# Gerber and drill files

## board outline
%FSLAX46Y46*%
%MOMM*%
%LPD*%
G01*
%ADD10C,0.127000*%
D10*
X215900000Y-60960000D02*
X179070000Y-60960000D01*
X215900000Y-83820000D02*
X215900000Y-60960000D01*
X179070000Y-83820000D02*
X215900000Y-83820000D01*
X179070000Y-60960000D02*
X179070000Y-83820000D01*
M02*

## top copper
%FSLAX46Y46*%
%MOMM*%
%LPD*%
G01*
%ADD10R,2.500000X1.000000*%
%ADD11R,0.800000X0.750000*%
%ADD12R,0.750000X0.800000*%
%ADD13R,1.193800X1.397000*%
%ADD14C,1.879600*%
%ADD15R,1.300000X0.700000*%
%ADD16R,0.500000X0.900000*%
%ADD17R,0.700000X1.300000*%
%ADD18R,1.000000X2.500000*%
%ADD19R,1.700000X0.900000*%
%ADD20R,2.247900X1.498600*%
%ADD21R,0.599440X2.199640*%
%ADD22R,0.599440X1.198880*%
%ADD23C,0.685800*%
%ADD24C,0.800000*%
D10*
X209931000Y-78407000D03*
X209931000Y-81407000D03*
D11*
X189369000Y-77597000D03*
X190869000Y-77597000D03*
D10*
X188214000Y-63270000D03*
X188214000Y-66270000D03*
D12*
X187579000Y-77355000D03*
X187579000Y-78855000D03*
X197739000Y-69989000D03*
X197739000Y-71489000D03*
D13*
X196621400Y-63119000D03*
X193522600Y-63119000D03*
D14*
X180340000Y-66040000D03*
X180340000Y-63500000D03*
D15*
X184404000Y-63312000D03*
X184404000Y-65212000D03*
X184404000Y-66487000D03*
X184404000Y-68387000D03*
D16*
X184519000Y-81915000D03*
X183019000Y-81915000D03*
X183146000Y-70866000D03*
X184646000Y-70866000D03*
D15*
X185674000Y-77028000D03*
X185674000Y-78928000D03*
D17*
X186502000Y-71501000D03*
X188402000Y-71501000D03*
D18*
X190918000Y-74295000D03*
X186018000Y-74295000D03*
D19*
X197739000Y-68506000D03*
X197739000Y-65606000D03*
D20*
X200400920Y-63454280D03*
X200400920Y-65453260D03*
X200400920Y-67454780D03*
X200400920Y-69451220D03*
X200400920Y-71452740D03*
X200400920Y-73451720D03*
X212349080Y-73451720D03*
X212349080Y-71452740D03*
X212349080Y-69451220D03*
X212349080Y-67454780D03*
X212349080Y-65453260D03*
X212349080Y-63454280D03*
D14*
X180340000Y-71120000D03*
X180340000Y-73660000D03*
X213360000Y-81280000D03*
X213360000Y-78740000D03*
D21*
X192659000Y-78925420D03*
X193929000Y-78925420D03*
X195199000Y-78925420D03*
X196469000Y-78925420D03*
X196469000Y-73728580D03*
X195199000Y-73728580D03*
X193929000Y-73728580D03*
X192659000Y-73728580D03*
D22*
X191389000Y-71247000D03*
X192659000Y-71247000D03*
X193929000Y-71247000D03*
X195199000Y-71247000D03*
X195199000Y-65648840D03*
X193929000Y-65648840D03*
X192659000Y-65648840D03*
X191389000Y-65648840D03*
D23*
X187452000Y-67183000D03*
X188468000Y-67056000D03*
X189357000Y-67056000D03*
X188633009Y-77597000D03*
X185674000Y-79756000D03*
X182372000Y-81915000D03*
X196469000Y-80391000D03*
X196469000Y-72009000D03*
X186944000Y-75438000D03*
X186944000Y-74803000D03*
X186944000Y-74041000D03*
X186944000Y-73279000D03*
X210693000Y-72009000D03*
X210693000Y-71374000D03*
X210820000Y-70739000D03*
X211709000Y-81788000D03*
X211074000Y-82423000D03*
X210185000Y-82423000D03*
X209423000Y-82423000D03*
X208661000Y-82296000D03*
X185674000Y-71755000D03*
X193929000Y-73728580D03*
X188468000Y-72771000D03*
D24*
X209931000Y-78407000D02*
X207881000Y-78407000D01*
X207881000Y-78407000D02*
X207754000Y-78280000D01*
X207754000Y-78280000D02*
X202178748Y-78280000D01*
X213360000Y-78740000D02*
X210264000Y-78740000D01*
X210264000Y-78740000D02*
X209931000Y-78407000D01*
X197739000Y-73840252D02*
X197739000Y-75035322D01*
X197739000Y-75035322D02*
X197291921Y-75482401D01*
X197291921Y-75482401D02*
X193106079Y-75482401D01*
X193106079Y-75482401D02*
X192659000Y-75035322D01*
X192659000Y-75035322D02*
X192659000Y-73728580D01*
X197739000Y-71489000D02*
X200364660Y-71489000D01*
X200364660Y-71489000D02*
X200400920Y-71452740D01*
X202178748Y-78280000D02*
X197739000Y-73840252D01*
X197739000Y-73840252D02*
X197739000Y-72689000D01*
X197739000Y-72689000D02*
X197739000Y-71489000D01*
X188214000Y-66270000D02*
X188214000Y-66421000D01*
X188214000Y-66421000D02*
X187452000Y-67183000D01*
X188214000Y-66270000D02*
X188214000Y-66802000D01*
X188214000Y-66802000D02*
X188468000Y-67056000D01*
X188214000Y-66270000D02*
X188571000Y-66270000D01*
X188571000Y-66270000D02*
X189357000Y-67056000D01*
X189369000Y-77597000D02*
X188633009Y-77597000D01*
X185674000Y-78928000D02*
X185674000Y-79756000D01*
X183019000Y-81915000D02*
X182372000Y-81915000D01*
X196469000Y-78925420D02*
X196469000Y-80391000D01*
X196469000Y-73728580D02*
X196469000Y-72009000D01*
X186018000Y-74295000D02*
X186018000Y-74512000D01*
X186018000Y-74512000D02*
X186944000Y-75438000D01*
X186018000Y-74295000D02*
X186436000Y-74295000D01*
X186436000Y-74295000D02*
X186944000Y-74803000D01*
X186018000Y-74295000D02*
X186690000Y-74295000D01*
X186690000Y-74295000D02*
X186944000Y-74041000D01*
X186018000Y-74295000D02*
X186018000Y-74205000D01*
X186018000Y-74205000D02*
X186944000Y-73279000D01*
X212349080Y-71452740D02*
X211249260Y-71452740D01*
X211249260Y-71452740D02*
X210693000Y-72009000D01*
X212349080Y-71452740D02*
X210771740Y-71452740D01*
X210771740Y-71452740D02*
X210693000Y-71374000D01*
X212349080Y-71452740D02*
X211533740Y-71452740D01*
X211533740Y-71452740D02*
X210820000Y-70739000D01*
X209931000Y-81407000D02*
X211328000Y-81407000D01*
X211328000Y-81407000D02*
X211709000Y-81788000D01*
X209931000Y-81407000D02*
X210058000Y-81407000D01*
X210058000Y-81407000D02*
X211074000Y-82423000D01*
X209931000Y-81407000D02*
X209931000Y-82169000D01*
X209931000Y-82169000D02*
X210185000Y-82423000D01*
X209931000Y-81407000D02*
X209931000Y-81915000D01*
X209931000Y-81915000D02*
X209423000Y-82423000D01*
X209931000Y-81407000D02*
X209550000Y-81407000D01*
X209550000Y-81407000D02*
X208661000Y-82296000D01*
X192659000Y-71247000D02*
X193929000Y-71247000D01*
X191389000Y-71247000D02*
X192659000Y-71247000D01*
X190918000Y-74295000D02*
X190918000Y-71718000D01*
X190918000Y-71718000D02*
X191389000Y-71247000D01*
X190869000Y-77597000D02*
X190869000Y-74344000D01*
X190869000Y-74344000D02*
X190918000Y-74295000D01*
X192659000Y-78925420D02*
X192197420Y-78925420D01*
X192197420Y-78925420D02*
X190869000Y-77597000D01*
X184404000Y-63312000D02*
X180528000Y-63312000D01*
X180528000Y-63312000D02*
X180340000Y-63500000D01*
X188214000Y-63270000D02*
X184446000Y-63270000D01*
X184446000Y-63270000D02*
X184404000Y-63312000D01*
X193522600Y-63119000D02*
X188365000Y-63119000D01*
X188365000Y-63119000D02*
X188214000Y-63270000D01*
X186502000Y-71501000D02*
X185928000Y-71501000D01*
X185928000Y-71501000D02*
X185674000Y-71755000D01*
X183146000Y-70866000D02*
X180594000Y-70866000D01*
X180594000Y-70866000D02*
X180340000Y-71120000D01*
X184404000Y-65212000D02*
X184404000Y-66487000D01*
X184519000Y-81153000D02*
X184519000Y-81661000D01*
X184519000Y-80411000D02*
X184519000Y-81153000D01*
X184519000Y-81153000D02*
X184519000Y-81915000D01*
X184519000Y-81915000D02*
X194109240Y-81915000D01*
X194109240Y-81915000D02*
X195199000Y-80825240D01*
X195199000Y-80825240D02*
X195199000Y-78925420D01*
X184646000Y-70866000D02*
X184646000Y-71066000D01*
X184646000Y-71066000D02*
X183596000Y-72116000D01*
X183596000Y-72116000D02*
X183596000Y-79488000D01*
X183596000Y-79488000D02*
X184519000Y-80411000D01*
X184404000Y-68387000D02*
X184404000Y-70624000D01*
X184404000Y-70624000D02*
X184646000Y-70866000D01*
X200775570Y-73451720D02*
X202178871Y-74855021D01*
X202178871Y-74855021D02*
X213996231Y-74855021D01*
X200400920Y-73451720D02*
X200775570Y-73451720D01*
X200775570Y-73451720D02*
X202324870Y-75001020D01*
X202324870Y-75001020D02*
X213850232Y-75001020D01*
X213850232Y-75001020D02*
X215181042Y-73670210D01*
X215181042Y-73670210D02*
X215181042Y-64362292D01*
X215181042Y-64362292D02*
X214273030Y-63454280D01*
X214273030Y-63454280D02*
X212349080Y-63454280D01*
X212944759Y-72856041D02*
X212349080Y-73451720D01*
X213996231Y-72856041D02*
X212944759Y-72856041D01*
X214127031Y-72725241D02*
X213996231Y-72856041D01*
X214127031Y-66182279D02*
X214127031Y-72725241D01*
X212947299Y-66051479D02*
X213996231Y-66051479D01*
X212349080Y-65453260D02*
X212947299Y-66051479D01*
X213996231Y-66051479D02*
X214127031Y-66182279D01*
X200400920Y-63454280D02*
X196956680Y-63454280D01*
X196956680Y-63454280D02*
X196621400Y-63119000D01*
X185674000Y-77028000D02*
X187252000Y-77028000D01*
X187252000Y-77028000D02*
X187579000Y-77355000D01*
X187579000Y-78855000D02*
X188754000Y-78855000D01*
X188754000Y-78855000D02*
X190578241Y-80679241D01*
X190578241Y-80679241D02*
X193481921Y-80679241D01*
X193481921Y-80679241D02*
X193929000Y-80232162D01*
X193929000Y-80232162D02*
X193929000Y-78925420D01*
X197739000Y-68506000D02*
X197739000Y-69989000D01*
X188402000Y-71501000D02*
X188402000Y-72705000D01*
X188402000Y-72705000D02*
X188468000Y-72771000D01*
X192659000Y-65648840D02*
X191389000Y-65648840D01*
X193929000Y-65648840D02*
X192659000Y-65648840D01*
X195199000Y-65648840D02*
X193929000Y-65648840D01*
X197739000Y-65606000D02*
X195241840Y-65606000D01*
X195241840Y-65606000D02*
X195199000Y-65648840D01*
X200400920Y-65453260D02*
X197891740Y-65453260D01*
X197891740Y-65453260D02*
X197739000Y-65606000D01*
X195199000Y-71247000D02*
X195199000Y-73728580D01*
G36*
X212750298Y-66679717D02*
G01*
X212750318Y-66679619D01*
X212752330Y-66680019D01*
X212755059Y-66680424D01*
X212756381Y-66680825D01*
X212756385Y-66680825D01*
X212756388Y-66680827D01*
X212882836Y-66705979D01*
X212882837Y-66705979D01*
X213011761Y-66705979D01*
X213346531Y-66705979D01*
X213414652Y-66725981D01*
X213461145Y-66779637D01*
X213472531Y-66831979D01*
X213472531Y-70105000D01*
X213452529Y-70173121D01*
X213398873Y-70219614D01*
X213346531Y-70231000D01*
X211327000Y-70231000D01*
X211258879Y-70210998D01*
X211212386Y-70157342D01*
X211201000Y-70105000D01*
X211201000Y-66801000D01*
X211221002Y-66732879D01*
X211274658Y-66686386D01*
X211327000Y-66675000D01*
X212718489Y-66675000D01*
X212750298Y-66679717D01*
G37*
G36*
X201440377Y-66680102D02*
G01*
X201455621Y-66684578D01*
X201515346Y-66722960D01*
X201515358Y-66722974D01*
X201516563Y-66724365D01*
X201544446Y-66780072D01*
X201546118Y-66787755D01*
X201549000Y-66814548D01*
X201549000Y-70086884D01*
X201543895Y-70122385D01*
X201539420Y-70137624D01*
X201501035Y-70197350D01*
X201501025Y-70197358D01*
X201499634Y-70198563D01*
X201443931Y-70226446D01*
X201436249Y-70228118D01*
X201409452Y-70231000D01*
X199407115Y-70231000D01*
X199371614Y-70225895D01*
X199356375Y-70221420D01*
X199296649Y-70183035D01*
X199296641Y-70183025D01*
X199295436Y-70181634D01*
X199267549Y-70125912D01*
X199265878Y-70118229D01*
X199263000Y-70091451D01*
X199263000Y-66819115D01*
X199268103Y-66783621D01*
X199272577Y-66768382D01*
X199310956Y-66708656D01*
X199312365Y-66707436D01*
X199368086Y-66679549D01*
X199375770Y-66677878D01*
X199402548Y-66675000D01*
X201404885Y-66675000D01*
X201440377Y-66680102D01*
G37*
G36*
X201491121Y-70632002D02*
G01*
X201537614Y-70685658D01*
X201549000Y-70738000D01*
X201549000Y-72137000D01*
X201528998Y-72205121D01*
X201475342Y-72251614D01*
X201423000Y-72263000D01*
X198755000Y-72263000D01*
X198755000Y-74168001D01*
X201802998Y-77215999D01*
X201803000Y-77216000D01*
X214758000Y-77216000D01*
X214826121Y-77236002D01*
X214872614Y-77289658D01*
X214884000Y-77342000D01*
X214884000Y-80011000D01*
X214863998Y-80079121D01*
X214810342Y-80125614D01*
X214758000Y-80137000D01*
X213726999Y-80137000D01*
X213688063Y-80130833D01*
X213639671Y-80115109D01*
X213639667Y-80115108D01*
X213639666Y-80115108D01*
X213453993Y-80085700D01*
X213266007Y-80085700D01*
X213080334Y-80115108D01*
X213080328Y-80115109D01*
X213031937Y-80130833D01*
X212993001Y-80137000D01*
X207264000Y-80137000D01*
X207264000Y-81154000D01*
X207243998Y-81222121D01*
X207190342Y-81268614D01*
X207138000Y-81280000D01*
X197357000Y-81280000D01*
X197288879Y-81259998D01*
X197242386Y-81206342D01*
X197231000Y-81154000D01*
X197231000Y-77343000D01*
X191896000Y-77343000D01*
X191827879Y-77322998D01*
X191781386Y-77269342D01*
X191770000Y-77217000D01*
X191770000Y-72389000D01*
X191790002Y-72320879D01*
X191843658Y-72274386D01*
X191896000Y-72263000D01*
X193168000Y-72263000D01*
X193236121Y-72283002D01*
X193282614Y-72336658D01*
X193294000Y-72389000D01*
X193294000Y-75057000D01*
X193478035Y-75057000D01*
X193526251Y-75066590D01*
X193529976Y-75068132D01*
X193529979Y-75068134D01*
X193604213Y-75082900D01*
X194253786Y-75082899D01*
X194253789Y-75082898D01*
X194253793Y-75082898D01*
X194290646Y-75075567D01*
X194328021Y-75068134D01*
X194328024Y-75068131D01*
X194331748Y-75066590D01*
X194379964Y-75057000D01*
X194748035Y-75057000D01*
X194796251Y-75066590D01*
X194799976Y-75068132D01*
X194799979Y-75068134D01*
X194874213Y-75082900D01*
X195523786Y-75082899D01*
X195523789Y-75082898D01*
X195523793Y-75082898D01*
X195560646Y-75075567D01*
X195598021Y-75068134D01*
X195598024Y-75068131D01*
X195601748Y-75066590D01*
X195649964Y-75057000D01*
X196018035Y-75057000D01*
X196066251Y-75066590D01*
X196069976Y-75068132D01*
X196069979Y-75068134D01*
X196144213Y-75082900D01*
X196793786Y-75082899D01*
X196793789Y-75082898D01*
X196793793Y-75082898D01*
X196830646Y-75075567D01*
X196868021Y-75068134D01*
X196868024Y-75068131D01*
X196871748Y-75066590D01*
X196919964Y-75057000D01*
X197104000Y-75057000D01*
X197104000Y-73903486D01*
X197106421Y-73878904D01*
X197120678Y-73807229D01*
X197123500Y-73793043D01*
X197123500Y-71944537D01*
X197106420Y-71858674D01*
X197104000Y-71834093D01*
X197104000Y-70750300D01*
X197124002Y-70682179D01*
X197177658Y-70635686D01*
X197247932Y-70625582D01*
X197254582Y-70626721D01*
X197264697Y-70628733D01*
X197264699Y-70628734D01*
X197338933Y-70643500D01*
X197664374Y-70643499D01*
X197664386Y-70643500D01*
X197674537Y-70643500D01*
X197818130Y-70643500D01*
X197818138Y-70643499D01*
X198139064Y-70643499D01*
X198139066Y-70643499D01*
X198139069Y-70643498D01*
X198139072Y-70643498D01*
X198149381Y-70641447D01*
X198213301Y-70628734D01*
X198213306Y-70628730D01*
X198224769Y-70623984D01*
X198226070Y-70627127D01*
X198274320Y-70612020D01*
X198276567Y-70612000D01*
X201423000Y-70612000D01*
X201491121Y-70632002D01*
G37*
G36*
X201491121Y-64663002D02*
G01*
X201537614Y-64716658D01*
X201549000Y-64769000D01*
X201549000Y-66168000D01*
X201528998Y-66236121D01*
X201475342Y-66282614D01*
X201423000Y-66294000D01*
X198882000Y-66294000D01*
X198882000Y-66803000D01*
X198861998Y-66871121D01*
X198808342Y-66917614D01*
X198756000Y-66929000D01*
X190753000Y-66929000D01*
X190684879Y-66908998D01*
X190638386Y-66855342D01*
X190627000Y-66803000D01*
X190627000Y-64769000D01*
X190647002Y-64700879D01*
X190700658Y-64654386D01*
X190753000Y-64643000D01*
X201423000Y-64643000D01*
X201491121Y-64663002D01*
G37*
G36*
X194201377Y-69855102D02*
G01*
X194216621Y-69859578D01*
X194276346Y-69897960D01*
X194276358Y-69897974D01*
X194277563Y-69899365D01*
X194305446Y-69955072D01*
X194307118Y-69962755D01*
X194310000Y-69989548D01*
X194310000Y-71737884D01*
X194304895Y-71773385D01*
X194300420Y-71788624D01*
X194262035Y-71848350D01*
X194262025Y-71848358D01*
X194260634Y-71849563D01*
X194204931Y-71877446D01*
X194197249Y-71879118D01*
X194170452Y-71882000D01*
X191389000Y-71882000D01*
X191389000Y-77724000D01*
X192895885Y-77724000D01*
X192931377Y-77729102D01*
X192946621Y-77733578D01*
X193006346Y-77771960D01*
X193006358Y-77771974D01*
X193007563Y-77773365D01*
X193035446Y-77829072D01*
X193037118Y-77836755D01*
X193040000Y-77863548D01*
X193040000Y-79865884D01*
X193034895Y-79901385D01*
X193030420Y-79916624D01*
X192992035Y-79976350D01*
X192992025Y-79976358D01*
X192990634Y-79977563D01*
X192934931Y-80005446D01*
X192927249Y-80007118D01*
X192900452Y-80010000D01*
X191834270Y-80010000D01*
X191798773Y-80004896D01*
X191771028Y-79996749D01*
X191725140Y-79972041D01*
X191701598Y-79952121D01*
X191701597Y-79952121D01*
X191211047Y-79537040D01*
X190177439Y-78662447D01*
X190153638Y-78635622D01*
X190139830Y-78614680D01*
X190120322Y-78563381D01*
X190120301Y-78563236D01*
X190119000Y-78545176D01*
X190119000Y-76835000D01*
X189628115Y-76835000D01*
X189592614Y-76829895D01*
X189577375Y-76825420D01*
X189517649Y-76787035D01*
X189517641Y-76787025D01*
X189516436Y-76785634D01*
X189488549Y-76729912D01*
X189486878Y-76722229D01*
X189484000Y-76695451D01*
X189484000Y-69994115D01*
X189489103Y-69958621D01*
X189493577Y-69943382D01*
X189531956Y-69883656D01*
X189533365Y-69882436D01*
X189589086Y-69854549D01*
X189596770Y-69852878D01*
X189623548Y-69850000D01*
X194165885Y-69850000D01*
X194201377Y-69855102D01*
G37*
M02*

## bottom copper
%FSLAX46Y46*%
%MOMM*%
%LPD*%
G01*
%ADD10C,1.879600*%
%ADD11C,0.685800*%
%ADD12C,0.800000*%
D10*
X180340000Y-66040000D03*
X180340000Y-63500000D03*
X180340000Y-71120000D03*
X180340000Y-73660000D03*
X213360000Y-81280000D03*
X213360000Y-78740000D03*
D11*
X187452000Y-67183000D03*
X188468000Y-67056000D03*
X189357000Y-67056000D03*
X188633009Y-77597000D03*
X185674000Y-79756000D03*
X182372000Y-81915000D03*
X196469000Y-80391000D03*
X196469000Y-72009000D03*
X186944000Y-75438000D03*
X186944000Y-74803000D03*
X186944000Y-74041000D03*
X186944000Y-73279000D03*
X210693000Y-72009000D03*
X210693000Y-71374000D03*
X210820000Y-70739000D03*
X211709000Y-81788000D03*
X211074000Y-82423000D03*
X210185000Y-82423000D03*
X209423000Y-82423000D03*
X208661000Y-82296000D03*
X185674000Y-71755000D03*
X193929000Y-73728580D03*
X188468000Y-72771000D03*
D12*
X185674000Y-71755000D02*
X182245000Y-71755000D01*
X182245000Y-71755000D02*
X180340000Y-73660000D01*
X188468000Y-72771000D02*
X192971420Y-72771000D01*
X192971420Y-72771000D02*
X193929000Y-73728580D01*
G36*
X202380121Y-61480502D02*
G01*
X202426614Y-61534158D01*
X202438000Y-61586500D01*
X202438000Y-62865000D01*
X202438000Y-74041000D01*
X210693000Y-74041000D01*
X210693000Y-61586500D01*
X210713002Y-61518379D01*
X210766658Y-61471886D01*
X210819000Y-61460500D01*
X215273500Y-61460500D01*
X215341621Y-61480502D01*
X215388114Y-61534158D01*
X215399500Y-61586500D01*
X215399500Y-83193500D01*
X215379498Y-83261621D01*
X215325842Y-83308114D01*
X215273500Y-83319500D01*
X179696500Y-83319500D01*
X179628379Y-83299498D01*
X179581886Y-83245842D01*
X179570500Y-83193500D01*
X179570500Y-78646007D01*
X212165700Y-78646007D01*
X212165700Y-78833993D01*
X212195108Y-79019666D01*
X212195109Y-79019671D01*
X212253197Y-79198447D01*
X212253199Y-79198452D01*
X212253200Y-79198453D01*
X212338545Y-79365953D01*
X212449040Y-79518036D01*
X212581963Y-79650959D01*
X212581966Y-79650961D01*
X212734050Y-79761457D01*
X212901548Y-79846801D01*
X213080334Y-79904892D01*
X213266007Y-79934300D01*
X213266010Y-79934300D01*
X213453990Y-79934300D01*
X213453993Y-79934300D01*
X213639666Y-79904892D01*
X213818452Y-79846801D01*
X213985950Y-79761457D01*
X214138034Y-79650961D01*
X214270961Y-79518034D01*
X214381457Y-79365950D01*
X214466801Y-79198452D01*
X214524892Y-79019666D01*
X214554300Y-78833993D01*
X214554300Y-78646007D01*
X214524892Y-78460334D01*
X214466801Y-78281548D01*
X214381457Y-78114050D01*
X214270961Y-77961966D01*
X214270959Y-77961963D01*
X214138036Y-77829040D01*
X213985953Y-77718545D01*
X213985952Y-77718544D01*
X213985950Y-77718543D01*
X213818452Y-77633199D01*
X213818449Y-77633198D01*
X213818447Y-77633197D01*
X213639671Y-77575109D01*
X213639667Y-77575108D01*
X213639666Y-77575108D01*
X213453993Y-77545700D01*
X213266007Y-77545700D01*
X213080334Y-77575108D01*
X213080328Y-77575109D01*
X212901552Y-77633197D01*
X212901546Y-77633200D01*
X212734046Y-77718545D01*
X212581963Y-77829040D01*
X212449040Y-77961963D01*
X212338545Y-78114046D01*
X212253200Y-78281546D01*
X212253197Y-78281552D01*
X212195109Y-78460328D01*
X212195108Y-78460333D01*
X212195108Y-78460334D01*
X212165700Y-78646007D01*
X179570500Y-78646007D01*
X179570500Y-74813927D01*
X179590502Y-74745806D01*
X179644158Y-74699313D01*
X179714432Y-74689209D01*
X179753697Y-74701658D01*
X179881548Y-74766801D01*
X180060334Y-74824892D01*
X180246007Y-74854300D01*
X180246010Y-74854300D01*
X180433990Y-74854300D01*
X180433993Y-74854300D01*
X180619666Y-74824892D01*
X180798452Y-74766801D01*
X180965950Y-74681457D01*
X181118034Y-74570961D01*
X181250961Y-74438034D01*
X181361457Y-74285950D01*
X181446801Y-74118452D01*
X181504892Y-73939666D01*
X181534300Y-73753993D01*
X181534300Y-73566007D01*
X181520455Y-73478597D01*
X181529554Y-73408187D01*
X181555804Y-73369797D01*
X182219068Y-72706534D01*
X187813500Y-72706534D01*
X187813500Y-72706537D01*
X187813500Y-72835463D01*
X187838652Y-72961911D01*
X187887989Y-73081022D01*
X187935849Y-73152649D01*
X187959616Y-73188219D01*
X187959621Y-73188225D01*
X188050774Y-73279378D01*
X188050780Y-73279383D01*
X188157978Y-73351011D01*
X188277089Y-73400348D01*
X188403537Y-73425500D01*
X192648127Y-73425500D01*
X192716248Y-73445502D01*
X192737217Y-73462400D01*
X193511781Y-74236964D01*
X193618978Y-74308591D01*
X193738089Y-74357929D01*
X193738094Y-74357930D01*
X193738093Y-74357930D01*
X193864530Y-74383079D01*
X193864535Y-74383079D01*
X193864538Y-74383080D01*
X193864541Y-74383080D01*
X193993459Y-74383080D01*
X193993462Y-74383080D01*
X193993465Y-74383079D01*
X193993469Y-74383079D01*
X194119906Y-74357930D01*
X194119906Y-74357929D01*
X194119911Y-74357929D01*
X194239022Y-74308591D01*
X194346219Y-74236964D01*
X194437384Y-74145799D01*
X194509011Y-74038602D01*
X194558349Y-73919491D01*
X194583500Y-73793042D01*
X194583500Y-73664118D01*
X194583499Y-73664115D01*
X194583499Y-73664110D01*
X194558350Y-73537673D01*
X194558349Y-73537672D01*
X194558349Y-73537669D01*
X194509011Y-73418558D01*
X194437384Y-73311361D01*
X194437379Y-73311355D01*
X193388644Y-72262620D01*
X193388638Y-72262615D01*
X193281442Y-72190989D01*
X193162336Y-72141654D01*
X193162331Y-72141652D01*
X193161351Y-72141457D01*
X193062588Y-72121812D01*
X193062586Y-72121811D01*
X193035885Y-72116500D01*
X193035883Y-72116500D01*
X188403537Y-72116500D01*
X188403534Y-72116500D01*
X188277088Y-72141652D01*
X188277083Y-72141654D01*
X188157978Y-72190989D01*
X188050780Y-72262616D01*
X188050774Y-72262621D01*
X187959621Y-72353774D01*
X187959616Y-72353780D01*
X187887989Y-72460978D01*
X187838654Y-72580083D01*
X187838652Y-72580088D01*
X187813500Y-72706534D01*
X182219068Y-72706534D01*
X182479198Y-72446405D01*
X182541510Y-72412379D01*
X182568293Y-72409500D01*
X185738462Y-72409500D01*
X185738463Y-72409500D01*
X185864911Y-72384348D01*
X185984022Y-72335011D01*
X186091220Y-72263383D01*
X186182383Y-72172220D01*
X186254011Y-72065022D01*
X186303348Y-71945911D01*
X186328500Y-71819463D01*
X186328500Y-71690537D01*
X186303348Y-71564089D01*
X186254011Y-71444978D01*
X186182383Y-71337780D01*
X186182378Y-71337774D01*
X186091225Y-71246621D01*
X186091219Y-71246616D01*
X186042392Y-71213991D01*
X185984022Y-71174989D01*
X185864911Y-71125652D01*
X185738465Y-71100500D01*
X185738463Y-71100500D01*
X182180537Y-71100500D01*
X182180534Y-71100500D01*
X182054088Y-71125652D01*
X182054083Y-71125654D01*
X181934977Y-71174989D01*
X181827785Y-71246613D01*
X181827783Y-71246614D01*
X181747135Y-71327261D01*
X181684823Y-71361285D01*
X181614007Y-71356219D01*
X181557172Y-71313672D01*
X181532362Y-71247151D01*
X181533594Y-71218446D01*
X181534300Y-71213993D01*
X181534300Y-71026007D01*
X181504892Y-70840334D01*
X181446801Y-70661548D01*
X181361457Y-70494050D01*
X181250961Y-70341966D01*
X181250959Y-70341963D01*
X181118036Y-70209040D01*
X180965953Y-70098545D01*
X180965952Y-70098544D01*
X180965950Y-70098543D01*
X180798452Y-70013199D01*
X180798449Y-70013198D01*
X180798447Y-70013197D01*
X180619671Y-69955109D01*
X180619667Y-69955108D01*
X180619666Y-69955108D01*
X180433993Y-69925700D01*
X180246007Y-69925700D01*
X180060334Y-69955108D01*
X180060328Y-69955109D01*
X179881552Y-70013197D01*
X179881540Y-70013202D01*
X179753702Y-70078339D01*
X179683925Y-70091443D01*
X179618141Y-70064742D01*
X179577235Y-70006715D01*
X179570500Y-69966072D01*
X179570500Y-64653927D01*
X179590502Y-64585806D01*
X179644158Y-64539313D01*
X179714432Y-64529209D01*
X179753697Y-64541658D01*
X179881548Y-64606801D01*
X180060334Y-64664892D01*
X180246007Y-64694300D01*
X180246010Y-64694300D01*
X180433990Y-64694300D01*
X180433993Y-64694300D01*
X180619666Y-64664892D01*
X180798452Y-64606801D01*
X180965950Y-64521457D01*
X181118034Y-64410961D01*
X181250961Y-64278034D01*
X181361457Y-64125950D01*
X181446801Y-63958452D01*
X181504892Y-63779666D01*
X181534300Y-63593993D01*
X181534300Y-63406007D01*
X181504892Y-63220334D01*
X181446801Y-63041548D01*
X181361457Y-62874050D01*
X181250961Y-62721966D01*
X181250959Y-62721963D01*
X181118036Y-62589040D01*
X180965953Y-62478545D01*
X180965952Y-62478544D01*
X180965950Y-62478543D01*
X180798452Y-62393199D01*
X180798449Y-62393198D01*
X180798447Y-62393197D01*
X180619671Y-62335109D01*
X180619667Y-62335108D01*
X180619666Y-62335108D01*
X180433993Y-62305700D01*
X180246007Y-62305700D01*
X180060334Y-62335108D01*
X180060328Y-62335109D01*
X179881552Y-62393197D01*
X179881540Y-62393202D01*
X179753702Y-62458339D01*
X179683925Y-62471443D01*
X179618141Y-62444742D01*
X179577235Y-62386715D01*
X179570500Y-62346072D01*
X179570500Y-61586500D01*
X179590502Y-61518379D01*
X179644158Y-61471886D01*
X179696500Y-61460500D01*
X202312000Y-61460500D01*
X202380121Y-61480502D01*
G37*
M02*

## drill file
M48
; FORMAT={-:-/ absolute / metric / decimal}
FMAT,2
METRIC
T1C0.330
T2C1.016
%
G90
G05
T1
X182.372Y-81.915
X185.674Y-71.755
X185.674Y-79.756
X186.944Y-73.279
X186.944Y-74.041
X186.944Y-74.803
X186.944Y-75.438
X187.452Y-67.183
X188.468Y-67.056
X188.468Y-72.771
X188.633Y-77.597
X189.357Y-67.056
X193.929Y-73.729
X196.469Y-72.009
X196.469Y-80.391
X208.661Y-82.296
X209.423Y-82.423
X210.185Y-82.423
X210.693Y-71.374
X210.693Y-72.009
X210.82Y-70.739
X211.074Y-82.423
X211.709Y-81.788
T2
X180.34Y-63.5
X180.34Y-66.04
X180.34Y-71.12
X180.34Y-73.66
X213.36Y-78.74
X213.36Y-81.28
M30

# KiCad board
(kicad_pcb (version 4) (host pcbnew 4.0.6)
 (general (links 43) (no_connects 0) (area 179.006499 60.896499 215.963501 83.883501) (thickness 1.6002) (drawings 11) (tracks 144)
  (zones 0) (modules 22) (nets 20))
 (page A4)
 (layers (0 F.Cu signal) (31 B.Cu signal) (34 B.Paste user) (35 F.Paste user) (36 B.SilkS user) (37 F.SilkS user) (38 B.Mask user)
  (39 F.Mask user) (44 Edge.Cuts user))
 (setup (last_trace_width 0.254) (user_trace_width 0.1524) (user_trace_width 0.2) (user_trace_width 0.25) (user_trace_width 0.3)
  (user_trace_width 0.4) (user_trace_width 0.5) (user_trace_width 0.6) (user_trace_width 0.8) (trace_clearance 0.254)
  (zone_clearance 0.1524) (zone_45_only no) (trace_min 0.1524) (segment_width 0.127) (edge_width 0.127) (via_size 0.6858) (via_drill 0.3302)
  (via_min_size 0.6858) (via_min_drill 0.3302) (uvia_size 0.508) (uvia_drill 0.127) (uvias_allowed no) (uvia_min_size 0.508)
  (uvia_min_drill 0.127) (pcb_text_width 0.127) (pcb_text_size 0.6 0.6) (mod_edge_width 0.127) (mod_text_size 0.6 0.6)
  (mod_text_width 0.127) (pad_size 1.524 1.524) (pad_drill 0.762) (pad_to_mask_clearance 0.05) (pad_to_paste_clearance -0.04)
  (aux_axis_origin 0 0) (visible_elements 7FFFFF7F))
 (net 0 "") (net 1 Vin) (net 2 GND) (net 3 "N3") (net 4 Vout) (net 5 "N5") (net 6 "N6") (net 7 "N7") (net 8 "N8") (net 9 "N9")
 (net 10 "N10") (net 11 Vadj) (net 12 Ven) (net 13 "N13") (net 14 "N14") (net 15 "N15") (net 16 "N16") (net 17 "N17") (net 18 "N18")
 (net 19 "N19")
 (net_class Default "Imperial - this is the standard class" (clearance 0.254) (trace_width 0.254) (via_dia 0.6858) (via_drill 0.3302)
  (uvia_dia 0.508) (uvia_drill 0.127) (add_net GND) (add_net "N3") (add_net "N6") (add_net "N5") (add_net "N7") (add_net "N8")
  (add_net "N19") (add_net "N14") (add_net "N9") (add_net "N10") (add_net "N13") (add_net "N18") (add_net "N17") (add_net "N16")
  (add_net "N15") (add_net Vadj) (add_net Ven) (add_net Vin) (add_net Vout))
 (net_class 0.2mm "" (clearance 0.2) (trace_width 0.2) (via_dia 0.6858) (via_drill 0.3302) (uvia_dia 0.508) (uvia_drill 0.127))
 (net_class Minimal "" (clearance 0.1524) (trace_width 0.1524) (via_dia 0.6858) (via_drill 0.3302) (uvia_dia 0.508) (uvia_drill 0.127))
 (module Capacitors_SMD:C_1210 (layer F.Cu) (at 209.931 79.907 270)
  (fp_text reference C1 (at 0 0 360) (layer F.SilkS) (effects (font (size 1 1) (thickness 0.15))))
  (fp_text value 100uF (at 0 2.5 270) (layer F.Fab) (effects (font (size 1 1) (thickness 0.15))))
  (pad 1 smd rect (at -1.5 0 270) (size 1 2.5) (layers F.Cu F.Paste F.Mask) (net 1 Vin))
  (pad 2 smd rect (at 1.5 0 270) (size 1 2.5) (layers F.Cu F.Paste F.Mask) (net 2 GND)))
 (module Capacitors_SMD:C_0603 (layer F.Cu) (at 190.119 77.597 180)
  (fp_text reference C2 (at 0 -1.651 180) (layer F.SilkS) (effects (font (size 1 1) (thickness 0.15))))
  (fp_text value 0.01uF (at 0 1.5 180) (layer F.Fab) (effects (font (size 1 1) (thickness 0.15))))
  (pad 2 smd rect (at 0.75 0 180) (size 0.8 0.75) (layers F.Cu F.Paste F.Mask) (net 2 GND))
  (pad 1 smd rect (at -0.75 0 180) (size 0.8 0.75) (layers F.Cu F.Paste F.Mask) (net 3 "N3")))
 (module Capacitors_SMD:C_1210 (layer F.Cu) (at 188.214 64.77 270)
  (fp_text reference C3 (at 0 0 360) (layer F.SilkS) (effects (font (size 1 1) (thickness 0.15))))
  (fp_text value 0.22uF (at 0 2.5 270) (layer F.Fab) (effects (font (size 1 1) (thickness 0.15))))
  (pad 1 smd rect (at -1.5 0 270) (size 1 2.5) (layers F.Cu F.Paste F.Mask) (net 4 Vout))
  (pad 2 smd rect (at 1.5 0 270) (size 1 2.5) (layers F.Cu F.Paste F.Mask) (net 2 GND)))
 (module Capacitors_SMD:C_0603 (layer F.Cu) (at 187.579 78.105 90)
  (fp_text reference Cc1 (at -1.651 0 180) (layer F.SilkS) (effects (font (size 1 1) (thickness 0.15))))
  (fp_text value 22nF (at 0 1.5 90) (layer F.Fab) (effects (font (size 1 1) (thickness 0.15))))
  (pad 2 smd rect (at 0.75 0 90) (size 0.8 0.75) (layers F.Cu F.Paste F.Mask) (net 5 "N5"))
  (pad 1 smd rect (at -0.75 0 90) (size 0.8 0.75) (layers F.Cu F.Paste F.Mask) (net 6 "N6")))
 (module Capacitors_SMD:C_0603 (layer F.Cu) (at 197.739 70.739 90)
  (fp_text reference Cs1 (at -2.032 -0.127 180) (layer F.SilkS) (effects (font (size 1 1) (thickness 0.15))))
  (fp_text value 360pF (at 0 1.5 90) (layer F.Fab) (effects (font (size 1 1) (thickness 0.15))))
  (pad 2 smd rect (at 0.75 0 90) (size 0.8 0.75) (layers F.Cu F.Paste F.Mask) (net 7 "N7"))
  (pad 1 smd rect (at -0.75 0 90) (size 0.8 0.75) (layers F.Cu F.Paste F.Mask) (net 1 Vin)))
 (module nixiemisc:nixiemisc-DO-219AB (layer F.Cu) (at 195.072 63.119)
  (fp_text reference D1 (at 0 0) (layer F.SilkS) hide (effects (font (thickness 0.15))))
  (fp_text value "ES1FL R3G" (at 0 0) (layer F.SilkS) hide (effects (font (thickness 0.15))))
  (pad A smd rect (at 1.5494 0 180) (size 1.1938 1.397) (layers F.Cu F.Paste F.Mask) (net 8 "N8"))
  (pad C smd rect (at -1.5494 0) (size 1.1938 1.397) (layers F.Cu F.Paste F.Mask) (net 4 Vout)))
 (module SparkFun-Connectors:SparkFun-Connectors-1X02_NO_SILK (layer F.Cu) (at 180.34 66.04 90)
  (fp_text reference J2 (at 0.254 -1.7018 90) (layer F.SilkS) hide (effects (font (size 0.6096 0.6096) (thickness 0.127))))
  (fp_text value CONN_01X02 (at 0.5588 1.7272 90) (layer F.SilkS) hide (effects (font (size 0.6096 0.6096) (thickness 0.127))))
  (pad 1 thru_hole circle (at 0 0 90) (size 1.8796 1.8796) (drill 1.016) (layers *.Cu *.Paste *.Mask) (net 2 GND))
  (pad 2 thru_hole circle (at 2.54 0 90) (size 1.8796 1.8796) (drill 1.016) (layers *.Cu *.Paste *.Mask) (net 4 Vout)))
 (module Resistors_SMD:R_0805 (layer F.Cu) (at 184.404 64.262 270)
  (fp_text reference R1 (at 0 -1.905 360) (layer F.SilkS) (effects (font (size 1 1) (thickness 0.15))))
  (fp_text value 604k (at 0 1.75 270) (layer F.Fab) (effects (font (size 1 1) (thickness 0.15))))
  (pad 1 smd rect (at -0.95 0 270) (size 0.7 1.3) (layers F.Cu F.Paste F.Mask) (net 4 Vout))
  (pad 2 smd rect (at 0.95 0 270) (size 0.7 1.3) (layers F.Cu F.Paste F.Mask) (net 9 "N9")))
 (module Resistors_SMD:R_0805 (layer F.Cu) (at 184.404 67.437 270)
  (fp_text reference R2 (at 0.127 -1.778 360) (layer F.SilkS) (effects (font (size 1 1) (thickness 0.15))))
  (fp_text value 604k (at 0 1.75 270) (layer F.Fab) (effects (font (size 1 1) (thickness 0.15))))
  (pad 1 smd rect (at -0.95 0 270) (size 0.7 1.3) (layers F.Cu F.Paste F.Mask) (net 9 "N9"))
  (pad 2 smd rect (at 0.95 0 270) (size 0.7 1.3) (layers F.Cu F.Paste F.Mask) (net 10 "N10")))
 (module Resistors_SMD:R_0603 (layer F.Cu) (at 183.769 81.915 180)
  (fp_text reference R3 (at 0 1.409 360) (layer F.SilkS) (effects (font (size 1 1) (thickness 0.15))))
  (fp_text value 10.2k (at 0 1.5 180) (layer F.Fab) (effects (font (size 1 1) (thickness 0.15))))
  (pad 1 smd rect (at -0.75 0 180) (size 0.5 0.9) (layers F.Cu F.Paste F.Mask) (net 10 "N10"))
  (pad 2 smd rect (at 0.75 0 180) (size 0.5 0.9) (layers F.Cu F.Paste F.Mask) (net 2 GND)))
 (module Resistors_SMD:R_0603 (layer F.Cu) (at 183.896 70.866)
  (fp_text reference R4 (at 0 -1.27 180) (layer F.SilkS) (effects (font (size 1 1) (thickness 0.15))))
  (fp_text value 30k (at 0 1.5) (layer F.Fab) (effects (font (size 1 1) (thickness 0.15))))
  (pad 1 smd rect (at -0.75 0) (size 0.5 0.9) (layers F.Cu F.Paste F.Mask) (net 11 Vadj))
  (pad 2 smd rect (at 0.75 0) (size 0.5 0.9) (layers F.Cu F.Paste F.Mask) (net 10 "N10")))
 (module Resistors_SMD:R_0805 (layer F.Cu) (at 185.674 77.978 270)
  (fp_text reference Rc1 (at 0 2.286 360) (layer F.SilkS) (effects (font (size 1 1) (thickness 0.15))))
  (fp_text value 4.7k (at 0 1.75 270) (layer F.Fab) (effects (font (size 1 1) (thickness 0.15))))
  (pad 1 smd rect (at -0.95 0 270) (size 0.7 1.3) (layers F.Cu F.Paste F.Mask) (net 5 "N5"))
  (pad 2 smd rect (at 0.95 0 270) (size 0.7 1.3) (layers F.Cu F.Paste F.Mask) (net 2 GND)))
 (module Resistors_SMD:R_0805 (layer F.Cu) (at 187.452 71.501)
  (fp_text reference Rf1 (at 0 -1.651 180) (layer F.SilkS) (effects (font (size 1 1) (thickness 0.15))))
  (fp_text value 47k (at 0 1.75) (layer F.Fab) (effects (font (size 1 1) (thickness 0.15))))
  (pad 1 smd rect (at -0.95 0) (size 0.7 1.3) (layers F.Cu F.Paste F.Mask) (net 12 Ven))
  (pad 2 smd rect (at 0.95 0) (size 0.7 1.3) (layers F.Cu F.Paste F.Mask) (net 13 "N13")))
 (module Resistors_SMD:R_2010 (layer F.Cu) (at 188.468 74.295 180)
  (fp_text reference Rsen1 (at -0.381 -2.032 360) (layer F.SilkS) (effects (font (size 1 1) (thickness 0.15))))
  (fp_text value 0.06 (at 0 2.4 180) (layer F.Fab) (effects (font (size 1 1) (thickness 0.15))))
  (pad 1 smd rect (at -2.45 0 180) (size 1 2.5) (layers F.Cu F.Paste F.Mask) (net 3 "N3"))
  (pad 2 smd rect (at 2.45 0 180) (size 1 2.5) (layers F.Cu F.Paste F.Mask) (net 2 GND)))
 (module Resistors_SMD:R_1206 (layer F.Cu) (at 197.739 67.056 90)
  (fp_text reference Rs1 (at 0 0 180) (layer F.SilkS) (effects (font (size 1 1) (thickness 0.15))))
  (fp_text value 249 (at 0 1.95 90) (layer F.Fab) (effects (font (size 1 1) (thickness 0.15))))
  (pad 1 smd rect (at -1.45 0 90) (size 0.9 1.7) (layers F.Cu F.Paste F.Mask) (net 7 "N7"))
  (pad 2 smd rect (at 1.45 0 90) (size 0.9 1.7) (layers F.Cu F.Paste F.Mask) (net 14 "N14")))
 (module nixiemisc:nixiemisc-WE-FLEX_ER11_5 (layer F.Cu) (at 206.375 68.453 90)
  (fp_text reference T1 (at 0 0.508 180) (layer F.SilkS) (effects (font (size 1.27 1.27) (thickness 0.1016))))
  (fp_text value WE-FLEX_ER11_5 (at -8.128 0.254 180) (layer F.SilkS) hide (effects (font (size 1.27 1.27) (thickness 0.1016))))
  (pad 1 smd rect (at 4.99872 -5.97408 270) (size 1.4986 2.2479) (layers F.Cu F.Paste F.Mask) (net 8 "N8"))
  (pad 2 smd rect (at 2.99974 -5.97408 270) (size 1.4986 2.2479) (layers F.Cu F.Paste F.Mask) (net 14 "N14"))
  (pad 3 smd rect (at 0.99822 -5.97408 270) (size 1.4986 2.2479) (layers F.Cu F.Paste F.Mask) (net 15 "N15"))
  (pad 4 smd rect (at -0.99822 -5.97408 270) (size 1.4986 2.2479) (layers F.Cu F.Paste F.Mask) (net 15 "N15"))
  (pad 5 smd rect (at -2.99974 -5.97408 270) (size 1.4986 2.2479) (layers F.Cu F.Paste F.Mask) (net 1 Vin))
  (pad 6 smd rect (at -4.99872 -5.97408 270) (size 1.4986 2.2479) (layers F.Cu F.Paste F.Mask) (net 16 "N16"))
  (pad 7 smd rect (at -4.99872 5.97408 270) (size 1.4986 2.2479) (layers F.Cu F.Paste F.Mask) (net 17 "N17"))
  (pad 8 smd rect (at -2.99974 5.97408 270) (size 1.4986 2.2479) (layers F.Cu F.Paste F.Mask) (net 2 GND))
  (pad 9 smd rect (at -0.99822 5.97408 270) (size 1.4986 2.2479) (layers F.Cu F.Paste F.Mask) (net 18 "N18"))
  (pad 10 smd rect (at 0.99822 5.97408 270) (size 1.4986 2.2479) (layers F.Cu F.Paste F.Mask) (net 18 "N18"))
  (pad 11 smd rect (at 2.99974 5.97408 270) (size 1.4986 2.2479) (layers F.Cu F.Paste F.Mask) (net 17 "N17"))
  (pad 12 smd rect (at 4.99872 5.97408 270) (size 1.4986 2.2479) (layers F.Cu F.Paste F.Mask) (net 16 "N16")))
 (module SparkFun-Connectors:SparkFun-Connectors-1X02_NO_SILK (layer F.Cu) (at 180.34 71.12 270)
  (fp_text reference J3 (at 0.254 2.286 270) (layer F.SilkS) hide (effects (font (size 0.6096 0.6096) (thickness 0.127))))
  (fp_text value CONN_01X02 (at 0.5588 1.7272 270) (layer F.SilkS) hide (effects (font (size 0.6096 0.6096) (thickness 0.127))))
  (pad 1 thru_hole circle (at 0 0 270) (size 1.8796 1.8796) (drill 1.016) (layers *.Cu *.Paste *.Mask) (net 11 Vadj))
  (pad 2 thru_hole circle (at 2.54 0 270) (size 1.8796 1.8796) (drill 1.016) (layers *.Cu *.Paste *.Mask) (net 12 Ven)))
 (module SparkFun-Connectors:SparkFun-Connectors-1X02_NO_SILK (layer F.Cu) (at 213.36 81.28 90)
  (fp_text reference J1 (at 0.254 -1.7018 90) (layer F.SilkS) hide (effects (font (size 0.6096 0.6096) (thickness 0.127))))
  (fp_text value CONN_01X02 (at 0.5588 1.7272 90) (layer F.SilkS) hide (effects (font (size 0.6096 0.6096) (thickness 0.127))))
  (pad 1 thru_hole circle (at 0 0 90) (size 1.8796 1.8796) (drill 1.016) (layers *.Cu *.Paste *.Mask) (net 2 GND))
  (pad 2 thru_hole circle (at 2.54 0 90) (size 1.8796 1.8796) (drill 1.016) (layers *.Cu *.Paste *.Mask) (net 1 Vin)))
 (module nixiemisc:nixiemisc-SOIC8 (layer F.Cu) (at 194.564 76.327)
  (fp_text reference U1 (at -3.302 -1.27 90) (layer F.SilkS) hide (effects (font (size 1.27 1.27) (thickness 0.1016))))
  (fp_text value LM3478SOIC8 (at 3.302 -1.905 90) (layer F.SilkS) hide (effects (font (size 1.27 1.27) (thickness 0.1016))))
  (pad 1 smd rect (at -1.905 2.59842) (size 0.59944 2.19964) (layers F.Cu F.Paste F.Mask) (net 3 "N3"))
  (pad 2 smd rect (at -0.635 2.59842) (size 0.59944 2.19964) (layers F.Cu F.Paste F.Mask) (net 6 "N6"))
  (pad 3 smd rect (at 0.635 2.59842) (size 0.59944 2.19964) (layers F.Cu F.Paste F.Mask) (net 10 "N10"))
  (pad 4 smd rect (at 1.905 2.59842) (size 0.59944 2.19964) (layers F.Cu F.Paste F.Mask) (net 2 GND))
  (pad 5 smd rect (at 1.905 -2.59842) (size 0.59944 2.19964) (layers F.Cu F.Paste F.Mask) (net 2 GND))
  (pad 6 smd rect (at 0.635 -2.59842) (size 0.59944 2.19964) (layers F.Cu F.Paste F.Mask) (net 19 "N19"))
  (pad 7 smd rect (at -0.635 -2.59842) (size 0.59944 2.19964) (layers F.Cu F.Paste F.Mask) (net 13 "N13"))
  (pad 8 smd rect (at -1.905 -2.59842) (size 0.59944 2.19964) (layers F.Cu F.Paste F.Mask) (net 1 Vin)))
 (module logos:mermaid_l (layer B.Cu) (at 205.867 79.629 180)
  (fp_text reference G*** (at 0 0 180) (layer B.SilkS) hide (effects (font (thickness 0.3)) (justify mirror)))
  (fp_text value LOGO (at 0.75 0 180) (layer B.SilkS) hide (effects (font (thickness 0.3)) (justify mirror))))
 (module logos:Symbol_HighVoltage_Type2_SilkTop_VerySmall (layer F.Cu) (at 201.422 79.502)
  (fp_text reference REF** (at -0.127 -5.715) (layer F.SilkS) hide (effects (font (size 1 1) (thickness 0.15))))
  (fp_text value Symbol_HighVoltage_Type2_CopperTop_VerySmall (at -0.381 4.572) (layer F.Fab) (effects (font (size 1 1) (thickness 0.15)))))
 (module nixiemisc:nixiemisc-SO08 (layer F.Cu) (at 193.294 68.44792)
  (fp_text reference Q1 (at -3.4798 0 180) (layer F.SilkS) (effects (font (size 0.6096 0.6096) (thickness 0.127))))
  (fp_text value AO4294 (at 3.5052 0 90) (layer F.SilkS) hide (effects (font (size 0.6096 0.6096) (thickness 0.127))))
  (pad 1 smd rect (at -1.905 2.79908) (size 0.59944 1.19888) (layers F.Cu F.Paste F.Mask) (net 3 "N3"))
  (pad 2 smd rect (at -0.635 2.79908) (size 0.59944 1.19888) (layers F.Cu F.Paste F.Mask) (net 3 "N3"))
  (pad 3 smd rect (at 0.635 2.79908) (size 0.59944 1.19888) (layers F.Cu F.Paste F.Mask) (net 3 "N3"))
  (pad 4 smd rect (at 1.905 2.79908) (size 0.59944 1.19888) (layers F.Cu F.Paste F.Mask) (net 19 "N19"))
  (pad 5 smd rect (at 1.905 -2.79908) (size 0.59944 1.19888) (layers F.Cu F.Paste F.Mask) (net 14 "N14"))
  (pad 6 smd rect (at 0.635 -2.79908) (size 0.59944 1.19888) (layers F.Cu F.Paste F.Mask) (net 14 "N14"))
  (pad 7 smd rect (at -0.635 -2.79908) (size 0.59944 1.19888) (layers F.Cu F.Paste F.Mask) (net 14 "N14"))
  (pad 8 smd rect (at -1.905 -2.79908) (size 0.59944 1.19888) (layers F.Cu F.Paste F.Mask) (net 14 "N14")))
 (gr_line (start 215.9 60.96) (end 179.07 60.96) (layer Edge.Cuts) (width 0.127))
 (gr_line (start 215.9 83.82) (end 215.9 60.96) (layer Edge.Cuts) (width 0.127))
 (gr_line (start 179.07 83.82) (end 215.9 83.82) (layer Edge.Cuts) (width 0.127))
 (gr_line (start 179.07 60.96) (end 179.07 83.82) (layer Edge.Cuts) (width 0.127))
 (segment (start 209.931 78.407) (end 207.881 78.407) (width 0.8) (layer F.Cu) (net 1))
 (segment (start 207.881 78.407) (end 207.754 78.28) (width 0.8) (layer F.Cu) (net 1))
 (segment (start 207.754 78.28) (end 202.178748 78.28) (width 0.8) (layer F.Cu) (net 1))
 (segment (start 213.36 78.74) (end 210.264 78.74) (width 0.8) (layer F.Cu) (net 1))
 (segment (start 210.264 78.74) (end 209.931 78.407) (width 0.8) (layer F.Cu) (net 1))
 (segment (start 197.739 73.840252) (end 197.739 75.035322) (width 0.8) (layer F.Cu) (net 1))
 (segment (start 197.739 75.035322) (end 197.291921 75.482401) (width 0.8) (layer F.Cu) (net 1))
 (segment (start 197.291921 75.482401) (end 193.106079 75.482401) (width 0.8) (layer F.Cu) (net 1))
 (segment (start 193.106079 75.482401) (end 192.659 75.035322) (width 0.8) (layer F.Cu) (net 1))
 (segment (start 192.659 75.035322) (end 192.659 73.72858) (width 0.8) (layer F.Cu) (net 1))
 (segment (start 197.739 71.489) (end 200.36466 71.489) (width 0.8) (layer F.Cu) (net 1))
 (segment (start 200.36466 71.489) (end 200.40092 71.45274) (width 0.8) (layer F.Cu) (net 1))
 (segment (start 202.178748 78.28) (end 197.739 73.840252) (width 0.8) (layer F.Cu) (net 1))
 (segment (start 197.739 73.840252) (end 197.739 72.689) (width 0.8) (layer F.Cu) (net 1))
 (segment (start 197.739 72.689) (end 197.739 71.489) (width 0.8) (layer F.Cu) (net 1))
 (segment (start 188.214 66.27) (end 188.214 66.421) (width 0.8) (layer F.Cu) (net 2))
 (segment (start 188.214 66.421) (end 187.452 67.183) (width 0.8) (layer F.Cu) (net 2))
 (via (at 187.452 67.183) (size 0.6858) (drill 0.3302) (layers F.Cu B.Cu) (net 2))
 (segment (start 188.214 66.27) (end 188.214 66.802) (width 0.8) (layer F.Cu) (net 2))
 (segment (start 188.214 66.802) (end 188.468 67.056) (width 0.8) (layer F.Cu) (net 2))
 (via (at 188.468 67.056) (size 0.6858) (drill 0.3302) (layers F.Cu B.Cu) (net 2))
 (segment (start 188.214 66.27) (end 188.571 66.27) (width 0.8) (layer F.Cu) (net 2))
 (segment (start 188.571 66.27) (end 189.357 67.056) (width 0.8) (layer F.Cu) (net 2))
 (via (at 189.357 67.056) (size 0.6858) (drill 0.3302) (layers F.Cu B.Cu) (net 2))
 (segment (start 189.369 77.597) (end 188.633009 77.597) (width 0.8) (layer F.Cu) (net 2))
 (via (at 188.633009 77.597) (size 0.6858) (drill 0.3302) (layers F.Cu B.Cu) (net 2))
 (segment (start 185.674 78.928) (end 185.674 79.756) (width 0.8) (layer F.Cu) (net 2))
 (via (at 185.674 79.756) (size 0.6858) (drill 0.3302) (layers F.Cu B.Cu) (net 2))
 (segment (start 183.019 81.915) (end 182.372 81.915) (width 0.8) (layer F.Cu) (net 2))
 (via (at 182.372 81.915) (size 0.6858) (drill 0.3302) (layers F.Cu B.Cu) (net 2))
 (segment (start 196.469 78.92542) (end 196.469 80.391) (width 0.8) (layer F.Cu) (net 2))
 (via (at 196.469 80.391) (size 0.6858) (drill 0.3302) (layers F.Cu B.Cu) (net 2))
 (segment (start 196.469 73.72858) (end 196.469 72.009) (width 0.8) (layer F.Cu) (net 2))
 (via (at 196.469 72.009) (size 0.6858) (drill 0.3302) (layers F.Cu B.Cu) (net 2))
 (segment (start 186.018 74.295) (end 186.018 74.512) (width 0.8) (layer F.Cu) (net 2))
 (segment (start 186.018 74.512) (end 186.944 75.438) (width 0.8) (layer F.Cu) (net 2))
 (via (at 186.944 75.438) (size 0.6858) (drill 0.3302) (layers F.Cu B.Cu) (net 2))
 (segment (start 186.018 74.295) (end 186.436 74.295) (width 0.8) (layer F.Cu) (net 2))
 (segment (start 186.436 74.295) (end 186.944 74.803) (width 0.8) (layer F.Cu) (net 2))
 (via (at 186.944 74.803) (size 0.6858) (drill 0.3302) (layers F.Cu B.Cu) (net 2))
 (segment (start 186.018 74.295) (end 186.69 74.295) (width 0.8) (layer F.Cu) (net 2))
 (segment (start 186.69 74.295) (end 186.944 74.041) (width 0.8) (layer F.Cu) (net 2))
 (via (at 186.944 74.041) (size 0.6858) (drill 0.3302) (layers F.Cu B.Cu) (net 2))
 (segment (start 186.018 74.295) (end 186.018 74.205) (width 0.8) (layer F.Cu) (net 2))
 (segment (start 186.018 74.205) (end 186.944 73.279) (width 0.8) (layer F.Cu) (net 2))
 (via (at 186.944 73.279) (size 0.6858) (drill 0.3302) (layers F.Cu B.Cu) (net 2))
 (segment (start 212.34908 71.45274) (end 211.24926 71.45274) (width 0.8) (layer F.Cu) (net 2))
 (via (at 210.693 72.009) (size 0.6858) (drill 0.3302) (layers F.Cu B.Cu) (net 2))
 (segment (start 211.24926 71.45274) (end 210.693 72.009) (width 0.8) (layer F.Cu) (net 2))
 (segment (start 212.34908 71.45274) (end 210.77174 71.45274) (width 0.8) (layer F.Cu) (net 2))
 (segment (start 210.77174 71.45274) (end 210.693 71.374) (width 0.8) (layer F.Cu) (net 2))
 (via (at 210.693 71.374) (size 0.6858) (drill 0.3302) (layers F.Cu B.Cu) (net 2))
 (segment (start 212.34908 71.45274) (end 211.53374 71.45274) (width 0.8) (layer F.Cu) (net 2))
 (segment (start 211.53374 71.45274) (end 210.82 70.739) (width 0.8) (layer F.Cu) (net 2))
 (via (at 210.82 70.739) (size 0.6858) (drill 0.3302) (layers F.Cu B.Cu) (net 2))
 (segment (start 209.931 81.407) (end 211.328 81.407) (width 0.8) (layer F.Cu) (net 2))
 (segment (start 211.328 81.407) (end 211.709 81.788) (width 0.8) (layer F.Cu) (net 2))
 (via (at 211.709 81.788) (size 0.6858) (drill 0.3302) (layers F.Cu B.Cu) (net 2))
 (segment (start 209.931 81.407) (end 210.058 81.407) (width 0.8) (layer F.Cu) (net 2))
 (segment (start 210.058 81.407) (end 211.074 82.423) (width 0.8) (layer F.Cu) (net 2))
 (via (at 211.074 82.423) (size 0.6858) (drill 0.3302) (layers F.Cu B.Cu) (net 2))
 (segment (start 209.931 81.407) (end 209.931 82.169) (width 0.8) (layer F.Cu) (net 2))
 (segment (start 209.931 82.169) (end 210.185 82.423) (width 0.8) (layer F.Cu) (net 2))
 (via (at 210.185 82.423) (size 0.6858) (drill 0.3302) (layers F.Cu B.Cu) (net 2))
 (segment (start 209.931 81.407) (end 209.931 81.915) (width 0.8) (layer F.Cu) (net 2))
 (segment (start 209.931 81.915) (end 209.423 82.423) (width 0.8) (layer F.Cu) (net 2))
 (via (at 209.423 82.423) (size 0.6858) (drill 0.3302) (layers F.Cu B.Cu) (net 2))
 (segment (start 209.931 81.407) (end 209.55 81.407) (width 0.8) (layer F.Cu) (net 2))
 (segment (start 209.55 81.407) (end 208.661 82.296) (width 0.8) (layer F.Cu) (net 2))
 (via (at 208.661 82.296) (size 0.6858) (drill 0.3302) (layers F.Cu B.Cu) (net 2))
 (segment (start 192.659 71.247) (end 193.929 71.247) (width 0.8) (layer F.Cu) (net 3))
 (segment (start 191.389 71.247) (end 192.659 71.247) (width 0.8) (layer F.Cu) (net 3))
 (segment (start 190.918 74.295) (end 190.918 71.718) (width 0.8) (layer F.Cu) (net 3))
 (segment (start 190.918 71.718) (end 191.389 71.247) (width 0.8) (layer F.Cu) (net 3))
 (segment (start 190.869 77.597) (end 190.869 74.344) (width 0.8) (layer F.Cu) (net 3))
 (segment (start 190.869 74.344) (end 190.918 74.295) (width 0.8) (layer F.Cu) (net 3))
 (segment (start 192.659 78.92542) (end 192.19742 78.92542) (width 0.8) (layer F.Cu) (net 3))
 (segment (start 192.19742 78.92542) (end 190.869 77.597) (width 0.8) (layer F.Cu) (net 3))
 (segment (start 184.404 63.312) (end 180.528 63.312) (width 0.8) (layer F.Cu) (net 4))
 (segment (start 180.528 63.312) (end 180.34 63.5) (width 0.8) (layer F.Cu) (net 4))
 (segment (start 188.214 63.27) (end 184.446 63.27) (width 0.8) (layer F.Cu) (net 4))
 (segment (start 184.446 63.27) (end 184.404 63.312) (width 0.8) (layer F.Cu) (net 4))
 (segment (start 193.5226 63.119) (end 188.365 63.119) (width 0.8) (layer F.Cu) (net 4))
 (segment (start 188.365 63.119) (end 188.214 63.27) (width 0.8) (layer F.Cu) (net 4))
 (segment (start 185.674 71.755) (end 182.245 71.755) (width 0.8) (layer B.Cu) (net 12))
 (segment (start 182.245 71.755) (end 180.34 73.66) (width 0.8) (layer B.Cu) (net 12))
 (segment (start 186.502 71.501) (end 185.928 71.501) (width 0.8) (layer F.Cu) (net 12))
 (segment (start 185.928 71.501) (end 185.674 71.755) (width 0.8) (layer F.Cu) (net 12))
 (via (at 185.674 71.755) (size 0.6858) (drill 0.3302) (layers F.Cu B.Cu) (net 12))
 (segment (start 183.146 70.866) (end 180.594 70.866) (width 0.8) (layer F.Cu) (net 11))
 (segment (start 180.594 70.866) (end 180.34 71.12) (width 0.8) (layer F.Cu) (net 11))
 (segment (start 184.404 65.212) (end 184.404 66.487) (width 0.8) (layer F.Cu) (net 9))
 (segment (start 184.519 81.153) (end 184.519 81.661) (width 0.8) (layer F.Cu) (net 10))
 (segment (start 184.519 80.411) (end 184.519 81.153) (width 0.8) (layer F.Cu) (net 10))
 (segment (start 184.519 81.153) (end 184.519 81.915) (width 0.8) (layer F.Cu) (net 10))
 (segment (start 184.519 81.915) (end 194.10924 81.915) (width 0.8) (layer F.Cu) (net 10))
 (segment (start 194.10924 81.915) (end 195.199 80.82524) (width 0.8) (layer F.Cu) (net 10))
 (segment (start 195.199 80.82524) (end 195.199 78.92542) (width 0.8) (layer F.Cu) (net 10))
 (segment (start 184.646 70.866) (end 184.646 71.066) (width 0.8) (layer F.Cu) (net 10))
 (segment (start 184.646 71.066) (end 183.596 72.116) (width 0.8) (layer F.Cu) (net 10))
 (segment (start 183.596 72.116) (end 183.596 79.488) (width 0.8) (layer F.Cu) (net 10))
 (segment (start 183.596 79.488) (end 184.519 80.411) (width 0.8) (layer F.Cu) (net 10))
 (segment (start 184.404 68.387) (end 184.404 70.624) (width 0.8) (layer F.Cu) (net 10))
 (segment (start 184.404 70.624) (end 184.646 70.866) (width 0.8) (layer F.Cu) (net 10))
 (segment (start 200.77557 73.45172) (end 202.178871 74.855021) (width 0.8) (layer F.Cu) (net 16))
 (segment (start 202.178871 74.855021) (end 213.996231 74.855021) (width 0.8) (layer F.Cu) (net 16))
 (segment (start 200.40092 73.45172) (end 200.77557 73.45172) (width 0.8) (layer F.Cu) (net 16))
 (segment (start 200.77557 73.45172) (end 202.32487 75.00102) (width 0.8) (layer F.Cu) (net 16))
 (segment (start 202.32487 75.00102) (end 213.850232 75.00102) (width 0.8) (layer F.Cu) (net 16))
 (segment (start 213.850232 75.00102) (end 215.181042 73.67021) (width 0.8) (layer F.Cu) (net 16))
 (segment (start 215.181042 73.67021) (end 215.181042 64.362292) (width 0.8) (layer F.Cu) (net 16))
 (segment (start 215.181042 64.362292) (end 214.27303 63.45428) (width 0.8) (layer F.Cu) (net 16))
 (segment (start 214.27303 63.45428) (end 212.34908 63.45428) (width 0.8) (layer F.Cu) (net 16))
 (segment (start 212.944759 72.856041) (end 212.34908 73.45172) (width 0.8) (layer F.Cu) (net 17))
 (segment (start 213.996231 72.856041) (end 212.944759 72.856041) (width 0.8) (layer F.Cu) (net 17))
 (segment (start 214.127031 72.725241) (end 213.996231 72.856041) (width 0.8) (layer F.Cu) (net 17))
 (segment (start 214.127031 66.182279) (end 214.127031 72.725241) (width 0.8) (layer F.Cu) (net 17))
 (segment (start 212.947299 66.051479) (end 213.996231 66.051479) (width 0.8) (layer F.Cu) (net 17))
 (segment (start 212.34908 65.45326) (end 212.947299 66.051479) (width 0.8) (layer F.Cu) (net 17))
 (segment (start 213.996231 66.051479) (end 214.127031 66.182279) (width 0.8) (layer F.Cu) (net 17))
 (segment (start 200.40092 63.45428) (end 196.95668 63.45428) (width 0.8) (layer F.Cu) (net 8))
 (segment (start 196.95668 63.45428) (end 196.6214 63.119) (width 0.8) (layer F.Cu) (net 8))
 (segment (start 185.674 77.028) (end 187.252 77.028) (width 0.8) (layer F.Cu) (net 5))
 (segment (start 187.252 77.028) (end 187.579 77.355) (width 0.8) (layer F.Cu) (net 5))
 (segment (start 187.579 78.855) (end 188.754 78.855) (width 0.8) (layer F.Cu) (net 6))
 (segment (start 188.754 78.855) (end 190.578241 80.679241) (width 0.8) (layer F.Cu) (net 6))
 (segment (start 190.578241 80.679241) (end 193.481921 80.679241) (width 0.8) (layer F.Cu) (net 6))
 (segment (start 193.481921 80.679241) (end 193.929 80.232162) (width 0.8) (layer F.Cu) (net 6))
 (segment (start 193.929 80.232162) (end 193.929 78.92542) (width 0.8) (layer F.Cu) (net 6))
 (segment (start 197.739 68.506) (end 197.739 69.989) (width 0.8) (layer F.Cu) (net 7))
 (segment (start 188.468 72.771) (end 192.97142 72.771) (width 0.8) (layer B.Cu) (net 13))
 (segment (start 192.97142 72.771) (end 193.929 73.72858) (width 0.8) (layer B.Cu) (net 13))
 (via (at 193.929 73.72858) (size 0.6858) (drill 0.3302) (layers F.Cu B.Cu) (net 13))
 (segment (start 188.402 71.501) (end 188.402 72.705) (width 0.8) (layer F.Cu) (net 13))
 (segment (start 188.402 72.705) (end 188.468 72.771) (width 0.8) (layer F.Cu) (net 13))
 (via (at 188.468 72.771) (size 0.6858) (drill 0.3302) (layers F.Cu B.Cu) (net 13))
 (segment (start 192.659 65.64884) (end 191.389 65.64884) (width 0.8) (layer F.Cu) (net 14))
 (segment (start 193.929 65.64884) (end 192.659 65.64884) (width 0.8) (layer F.Cu) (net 14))
 (segment (start 195.199 65.64884) (end 193.929 65.64884) (width 0.8) (layer F.Cu) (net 14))
 (segment (start 197.739 65.606) (end 195.24184 65.606) (width 0.8) (layer F.Cu) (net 14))
 (segment (start 195.24184 65.606) (end 195.199 65.64884) (width 0.8) (layer F.Cu) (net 14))
 (segment (start 200.40092 65.45326) (end 197.89174 65.45326) (width 0.8) (layer F.Cu) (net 14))
 (segment (start 197.89174 65.45326) (end 197.739 65.606) (width 0.8) (layer F.Cu) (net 14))
 (segment (start 195.199 71.247) (end 195.199 73.72858) (width 0.8) (layer F.Cu) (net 19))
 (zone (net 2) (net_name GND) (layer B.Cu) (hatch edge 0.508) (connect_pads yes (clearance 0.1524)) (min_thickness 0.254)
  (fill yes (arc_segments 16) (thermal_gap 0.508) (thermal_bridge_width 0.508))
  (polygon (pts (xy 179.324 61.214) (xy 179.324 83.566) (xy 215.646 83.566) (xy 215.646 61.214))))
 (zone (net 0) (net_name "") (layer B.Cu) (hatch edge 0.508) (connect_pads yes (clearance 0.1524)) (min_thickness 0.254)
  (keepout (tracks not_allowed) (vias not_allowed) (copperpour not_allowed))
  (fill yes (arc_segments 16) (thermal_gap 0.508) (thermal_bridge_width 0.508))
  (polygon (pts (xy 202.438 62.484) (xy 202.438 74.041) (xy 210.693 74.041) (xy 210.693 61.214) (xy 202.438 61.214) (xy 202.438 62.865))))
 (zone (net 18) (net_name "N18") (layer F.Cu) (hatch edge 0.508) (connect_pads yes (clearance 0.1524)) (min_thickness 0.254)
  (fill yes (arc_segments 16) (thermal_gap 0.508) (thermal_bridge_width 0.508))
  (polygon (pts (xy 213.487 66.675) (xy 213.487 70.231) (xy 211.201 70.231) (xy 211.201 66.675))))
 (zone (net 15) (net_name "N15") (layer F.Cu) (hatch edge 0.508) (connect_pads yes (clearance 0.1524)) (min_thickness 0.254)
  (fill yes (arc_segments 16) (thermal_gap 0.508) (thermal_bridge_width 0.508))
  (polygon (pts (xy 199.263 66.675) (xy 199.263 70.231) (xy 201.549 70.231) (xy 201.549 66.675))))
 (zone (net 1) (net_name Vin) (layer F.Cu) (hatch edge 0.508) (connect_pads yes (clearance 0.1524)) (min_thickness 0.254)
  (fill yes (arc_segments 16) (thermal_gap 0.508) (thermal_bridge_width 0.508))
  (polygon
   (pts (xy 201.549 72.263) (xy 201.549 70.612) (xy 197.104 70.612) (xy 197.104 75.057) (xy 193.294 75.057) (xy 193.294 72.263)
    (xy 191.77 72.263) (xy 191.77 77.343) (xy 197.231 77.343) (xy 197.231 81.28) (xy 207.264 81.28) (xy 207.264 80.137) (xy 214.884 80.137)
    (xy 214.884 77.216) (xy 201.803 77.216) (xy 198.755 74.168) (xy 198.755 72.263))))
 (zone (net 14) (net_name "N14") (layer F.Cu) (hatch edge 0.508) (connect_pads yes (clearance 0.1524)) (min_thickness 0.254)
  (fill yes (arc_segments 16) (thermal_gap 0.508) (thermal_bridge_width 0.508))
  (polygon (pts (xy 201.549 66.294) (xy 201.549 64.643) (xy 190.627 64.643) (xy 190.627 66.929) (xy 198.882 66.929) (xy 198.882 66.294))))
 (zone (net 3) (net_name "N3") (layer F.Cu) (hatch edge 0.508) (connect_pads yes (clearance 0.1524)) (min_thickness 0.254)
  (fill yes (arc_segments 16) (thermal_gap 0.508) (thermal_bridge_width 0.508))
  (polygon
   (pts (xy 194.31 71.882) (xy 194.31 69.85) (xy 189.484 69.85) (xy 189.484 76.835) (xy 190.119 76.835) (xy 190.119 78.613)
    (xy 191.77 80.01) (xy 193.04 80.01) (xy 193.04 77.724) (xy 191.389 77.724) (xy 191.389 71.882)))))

